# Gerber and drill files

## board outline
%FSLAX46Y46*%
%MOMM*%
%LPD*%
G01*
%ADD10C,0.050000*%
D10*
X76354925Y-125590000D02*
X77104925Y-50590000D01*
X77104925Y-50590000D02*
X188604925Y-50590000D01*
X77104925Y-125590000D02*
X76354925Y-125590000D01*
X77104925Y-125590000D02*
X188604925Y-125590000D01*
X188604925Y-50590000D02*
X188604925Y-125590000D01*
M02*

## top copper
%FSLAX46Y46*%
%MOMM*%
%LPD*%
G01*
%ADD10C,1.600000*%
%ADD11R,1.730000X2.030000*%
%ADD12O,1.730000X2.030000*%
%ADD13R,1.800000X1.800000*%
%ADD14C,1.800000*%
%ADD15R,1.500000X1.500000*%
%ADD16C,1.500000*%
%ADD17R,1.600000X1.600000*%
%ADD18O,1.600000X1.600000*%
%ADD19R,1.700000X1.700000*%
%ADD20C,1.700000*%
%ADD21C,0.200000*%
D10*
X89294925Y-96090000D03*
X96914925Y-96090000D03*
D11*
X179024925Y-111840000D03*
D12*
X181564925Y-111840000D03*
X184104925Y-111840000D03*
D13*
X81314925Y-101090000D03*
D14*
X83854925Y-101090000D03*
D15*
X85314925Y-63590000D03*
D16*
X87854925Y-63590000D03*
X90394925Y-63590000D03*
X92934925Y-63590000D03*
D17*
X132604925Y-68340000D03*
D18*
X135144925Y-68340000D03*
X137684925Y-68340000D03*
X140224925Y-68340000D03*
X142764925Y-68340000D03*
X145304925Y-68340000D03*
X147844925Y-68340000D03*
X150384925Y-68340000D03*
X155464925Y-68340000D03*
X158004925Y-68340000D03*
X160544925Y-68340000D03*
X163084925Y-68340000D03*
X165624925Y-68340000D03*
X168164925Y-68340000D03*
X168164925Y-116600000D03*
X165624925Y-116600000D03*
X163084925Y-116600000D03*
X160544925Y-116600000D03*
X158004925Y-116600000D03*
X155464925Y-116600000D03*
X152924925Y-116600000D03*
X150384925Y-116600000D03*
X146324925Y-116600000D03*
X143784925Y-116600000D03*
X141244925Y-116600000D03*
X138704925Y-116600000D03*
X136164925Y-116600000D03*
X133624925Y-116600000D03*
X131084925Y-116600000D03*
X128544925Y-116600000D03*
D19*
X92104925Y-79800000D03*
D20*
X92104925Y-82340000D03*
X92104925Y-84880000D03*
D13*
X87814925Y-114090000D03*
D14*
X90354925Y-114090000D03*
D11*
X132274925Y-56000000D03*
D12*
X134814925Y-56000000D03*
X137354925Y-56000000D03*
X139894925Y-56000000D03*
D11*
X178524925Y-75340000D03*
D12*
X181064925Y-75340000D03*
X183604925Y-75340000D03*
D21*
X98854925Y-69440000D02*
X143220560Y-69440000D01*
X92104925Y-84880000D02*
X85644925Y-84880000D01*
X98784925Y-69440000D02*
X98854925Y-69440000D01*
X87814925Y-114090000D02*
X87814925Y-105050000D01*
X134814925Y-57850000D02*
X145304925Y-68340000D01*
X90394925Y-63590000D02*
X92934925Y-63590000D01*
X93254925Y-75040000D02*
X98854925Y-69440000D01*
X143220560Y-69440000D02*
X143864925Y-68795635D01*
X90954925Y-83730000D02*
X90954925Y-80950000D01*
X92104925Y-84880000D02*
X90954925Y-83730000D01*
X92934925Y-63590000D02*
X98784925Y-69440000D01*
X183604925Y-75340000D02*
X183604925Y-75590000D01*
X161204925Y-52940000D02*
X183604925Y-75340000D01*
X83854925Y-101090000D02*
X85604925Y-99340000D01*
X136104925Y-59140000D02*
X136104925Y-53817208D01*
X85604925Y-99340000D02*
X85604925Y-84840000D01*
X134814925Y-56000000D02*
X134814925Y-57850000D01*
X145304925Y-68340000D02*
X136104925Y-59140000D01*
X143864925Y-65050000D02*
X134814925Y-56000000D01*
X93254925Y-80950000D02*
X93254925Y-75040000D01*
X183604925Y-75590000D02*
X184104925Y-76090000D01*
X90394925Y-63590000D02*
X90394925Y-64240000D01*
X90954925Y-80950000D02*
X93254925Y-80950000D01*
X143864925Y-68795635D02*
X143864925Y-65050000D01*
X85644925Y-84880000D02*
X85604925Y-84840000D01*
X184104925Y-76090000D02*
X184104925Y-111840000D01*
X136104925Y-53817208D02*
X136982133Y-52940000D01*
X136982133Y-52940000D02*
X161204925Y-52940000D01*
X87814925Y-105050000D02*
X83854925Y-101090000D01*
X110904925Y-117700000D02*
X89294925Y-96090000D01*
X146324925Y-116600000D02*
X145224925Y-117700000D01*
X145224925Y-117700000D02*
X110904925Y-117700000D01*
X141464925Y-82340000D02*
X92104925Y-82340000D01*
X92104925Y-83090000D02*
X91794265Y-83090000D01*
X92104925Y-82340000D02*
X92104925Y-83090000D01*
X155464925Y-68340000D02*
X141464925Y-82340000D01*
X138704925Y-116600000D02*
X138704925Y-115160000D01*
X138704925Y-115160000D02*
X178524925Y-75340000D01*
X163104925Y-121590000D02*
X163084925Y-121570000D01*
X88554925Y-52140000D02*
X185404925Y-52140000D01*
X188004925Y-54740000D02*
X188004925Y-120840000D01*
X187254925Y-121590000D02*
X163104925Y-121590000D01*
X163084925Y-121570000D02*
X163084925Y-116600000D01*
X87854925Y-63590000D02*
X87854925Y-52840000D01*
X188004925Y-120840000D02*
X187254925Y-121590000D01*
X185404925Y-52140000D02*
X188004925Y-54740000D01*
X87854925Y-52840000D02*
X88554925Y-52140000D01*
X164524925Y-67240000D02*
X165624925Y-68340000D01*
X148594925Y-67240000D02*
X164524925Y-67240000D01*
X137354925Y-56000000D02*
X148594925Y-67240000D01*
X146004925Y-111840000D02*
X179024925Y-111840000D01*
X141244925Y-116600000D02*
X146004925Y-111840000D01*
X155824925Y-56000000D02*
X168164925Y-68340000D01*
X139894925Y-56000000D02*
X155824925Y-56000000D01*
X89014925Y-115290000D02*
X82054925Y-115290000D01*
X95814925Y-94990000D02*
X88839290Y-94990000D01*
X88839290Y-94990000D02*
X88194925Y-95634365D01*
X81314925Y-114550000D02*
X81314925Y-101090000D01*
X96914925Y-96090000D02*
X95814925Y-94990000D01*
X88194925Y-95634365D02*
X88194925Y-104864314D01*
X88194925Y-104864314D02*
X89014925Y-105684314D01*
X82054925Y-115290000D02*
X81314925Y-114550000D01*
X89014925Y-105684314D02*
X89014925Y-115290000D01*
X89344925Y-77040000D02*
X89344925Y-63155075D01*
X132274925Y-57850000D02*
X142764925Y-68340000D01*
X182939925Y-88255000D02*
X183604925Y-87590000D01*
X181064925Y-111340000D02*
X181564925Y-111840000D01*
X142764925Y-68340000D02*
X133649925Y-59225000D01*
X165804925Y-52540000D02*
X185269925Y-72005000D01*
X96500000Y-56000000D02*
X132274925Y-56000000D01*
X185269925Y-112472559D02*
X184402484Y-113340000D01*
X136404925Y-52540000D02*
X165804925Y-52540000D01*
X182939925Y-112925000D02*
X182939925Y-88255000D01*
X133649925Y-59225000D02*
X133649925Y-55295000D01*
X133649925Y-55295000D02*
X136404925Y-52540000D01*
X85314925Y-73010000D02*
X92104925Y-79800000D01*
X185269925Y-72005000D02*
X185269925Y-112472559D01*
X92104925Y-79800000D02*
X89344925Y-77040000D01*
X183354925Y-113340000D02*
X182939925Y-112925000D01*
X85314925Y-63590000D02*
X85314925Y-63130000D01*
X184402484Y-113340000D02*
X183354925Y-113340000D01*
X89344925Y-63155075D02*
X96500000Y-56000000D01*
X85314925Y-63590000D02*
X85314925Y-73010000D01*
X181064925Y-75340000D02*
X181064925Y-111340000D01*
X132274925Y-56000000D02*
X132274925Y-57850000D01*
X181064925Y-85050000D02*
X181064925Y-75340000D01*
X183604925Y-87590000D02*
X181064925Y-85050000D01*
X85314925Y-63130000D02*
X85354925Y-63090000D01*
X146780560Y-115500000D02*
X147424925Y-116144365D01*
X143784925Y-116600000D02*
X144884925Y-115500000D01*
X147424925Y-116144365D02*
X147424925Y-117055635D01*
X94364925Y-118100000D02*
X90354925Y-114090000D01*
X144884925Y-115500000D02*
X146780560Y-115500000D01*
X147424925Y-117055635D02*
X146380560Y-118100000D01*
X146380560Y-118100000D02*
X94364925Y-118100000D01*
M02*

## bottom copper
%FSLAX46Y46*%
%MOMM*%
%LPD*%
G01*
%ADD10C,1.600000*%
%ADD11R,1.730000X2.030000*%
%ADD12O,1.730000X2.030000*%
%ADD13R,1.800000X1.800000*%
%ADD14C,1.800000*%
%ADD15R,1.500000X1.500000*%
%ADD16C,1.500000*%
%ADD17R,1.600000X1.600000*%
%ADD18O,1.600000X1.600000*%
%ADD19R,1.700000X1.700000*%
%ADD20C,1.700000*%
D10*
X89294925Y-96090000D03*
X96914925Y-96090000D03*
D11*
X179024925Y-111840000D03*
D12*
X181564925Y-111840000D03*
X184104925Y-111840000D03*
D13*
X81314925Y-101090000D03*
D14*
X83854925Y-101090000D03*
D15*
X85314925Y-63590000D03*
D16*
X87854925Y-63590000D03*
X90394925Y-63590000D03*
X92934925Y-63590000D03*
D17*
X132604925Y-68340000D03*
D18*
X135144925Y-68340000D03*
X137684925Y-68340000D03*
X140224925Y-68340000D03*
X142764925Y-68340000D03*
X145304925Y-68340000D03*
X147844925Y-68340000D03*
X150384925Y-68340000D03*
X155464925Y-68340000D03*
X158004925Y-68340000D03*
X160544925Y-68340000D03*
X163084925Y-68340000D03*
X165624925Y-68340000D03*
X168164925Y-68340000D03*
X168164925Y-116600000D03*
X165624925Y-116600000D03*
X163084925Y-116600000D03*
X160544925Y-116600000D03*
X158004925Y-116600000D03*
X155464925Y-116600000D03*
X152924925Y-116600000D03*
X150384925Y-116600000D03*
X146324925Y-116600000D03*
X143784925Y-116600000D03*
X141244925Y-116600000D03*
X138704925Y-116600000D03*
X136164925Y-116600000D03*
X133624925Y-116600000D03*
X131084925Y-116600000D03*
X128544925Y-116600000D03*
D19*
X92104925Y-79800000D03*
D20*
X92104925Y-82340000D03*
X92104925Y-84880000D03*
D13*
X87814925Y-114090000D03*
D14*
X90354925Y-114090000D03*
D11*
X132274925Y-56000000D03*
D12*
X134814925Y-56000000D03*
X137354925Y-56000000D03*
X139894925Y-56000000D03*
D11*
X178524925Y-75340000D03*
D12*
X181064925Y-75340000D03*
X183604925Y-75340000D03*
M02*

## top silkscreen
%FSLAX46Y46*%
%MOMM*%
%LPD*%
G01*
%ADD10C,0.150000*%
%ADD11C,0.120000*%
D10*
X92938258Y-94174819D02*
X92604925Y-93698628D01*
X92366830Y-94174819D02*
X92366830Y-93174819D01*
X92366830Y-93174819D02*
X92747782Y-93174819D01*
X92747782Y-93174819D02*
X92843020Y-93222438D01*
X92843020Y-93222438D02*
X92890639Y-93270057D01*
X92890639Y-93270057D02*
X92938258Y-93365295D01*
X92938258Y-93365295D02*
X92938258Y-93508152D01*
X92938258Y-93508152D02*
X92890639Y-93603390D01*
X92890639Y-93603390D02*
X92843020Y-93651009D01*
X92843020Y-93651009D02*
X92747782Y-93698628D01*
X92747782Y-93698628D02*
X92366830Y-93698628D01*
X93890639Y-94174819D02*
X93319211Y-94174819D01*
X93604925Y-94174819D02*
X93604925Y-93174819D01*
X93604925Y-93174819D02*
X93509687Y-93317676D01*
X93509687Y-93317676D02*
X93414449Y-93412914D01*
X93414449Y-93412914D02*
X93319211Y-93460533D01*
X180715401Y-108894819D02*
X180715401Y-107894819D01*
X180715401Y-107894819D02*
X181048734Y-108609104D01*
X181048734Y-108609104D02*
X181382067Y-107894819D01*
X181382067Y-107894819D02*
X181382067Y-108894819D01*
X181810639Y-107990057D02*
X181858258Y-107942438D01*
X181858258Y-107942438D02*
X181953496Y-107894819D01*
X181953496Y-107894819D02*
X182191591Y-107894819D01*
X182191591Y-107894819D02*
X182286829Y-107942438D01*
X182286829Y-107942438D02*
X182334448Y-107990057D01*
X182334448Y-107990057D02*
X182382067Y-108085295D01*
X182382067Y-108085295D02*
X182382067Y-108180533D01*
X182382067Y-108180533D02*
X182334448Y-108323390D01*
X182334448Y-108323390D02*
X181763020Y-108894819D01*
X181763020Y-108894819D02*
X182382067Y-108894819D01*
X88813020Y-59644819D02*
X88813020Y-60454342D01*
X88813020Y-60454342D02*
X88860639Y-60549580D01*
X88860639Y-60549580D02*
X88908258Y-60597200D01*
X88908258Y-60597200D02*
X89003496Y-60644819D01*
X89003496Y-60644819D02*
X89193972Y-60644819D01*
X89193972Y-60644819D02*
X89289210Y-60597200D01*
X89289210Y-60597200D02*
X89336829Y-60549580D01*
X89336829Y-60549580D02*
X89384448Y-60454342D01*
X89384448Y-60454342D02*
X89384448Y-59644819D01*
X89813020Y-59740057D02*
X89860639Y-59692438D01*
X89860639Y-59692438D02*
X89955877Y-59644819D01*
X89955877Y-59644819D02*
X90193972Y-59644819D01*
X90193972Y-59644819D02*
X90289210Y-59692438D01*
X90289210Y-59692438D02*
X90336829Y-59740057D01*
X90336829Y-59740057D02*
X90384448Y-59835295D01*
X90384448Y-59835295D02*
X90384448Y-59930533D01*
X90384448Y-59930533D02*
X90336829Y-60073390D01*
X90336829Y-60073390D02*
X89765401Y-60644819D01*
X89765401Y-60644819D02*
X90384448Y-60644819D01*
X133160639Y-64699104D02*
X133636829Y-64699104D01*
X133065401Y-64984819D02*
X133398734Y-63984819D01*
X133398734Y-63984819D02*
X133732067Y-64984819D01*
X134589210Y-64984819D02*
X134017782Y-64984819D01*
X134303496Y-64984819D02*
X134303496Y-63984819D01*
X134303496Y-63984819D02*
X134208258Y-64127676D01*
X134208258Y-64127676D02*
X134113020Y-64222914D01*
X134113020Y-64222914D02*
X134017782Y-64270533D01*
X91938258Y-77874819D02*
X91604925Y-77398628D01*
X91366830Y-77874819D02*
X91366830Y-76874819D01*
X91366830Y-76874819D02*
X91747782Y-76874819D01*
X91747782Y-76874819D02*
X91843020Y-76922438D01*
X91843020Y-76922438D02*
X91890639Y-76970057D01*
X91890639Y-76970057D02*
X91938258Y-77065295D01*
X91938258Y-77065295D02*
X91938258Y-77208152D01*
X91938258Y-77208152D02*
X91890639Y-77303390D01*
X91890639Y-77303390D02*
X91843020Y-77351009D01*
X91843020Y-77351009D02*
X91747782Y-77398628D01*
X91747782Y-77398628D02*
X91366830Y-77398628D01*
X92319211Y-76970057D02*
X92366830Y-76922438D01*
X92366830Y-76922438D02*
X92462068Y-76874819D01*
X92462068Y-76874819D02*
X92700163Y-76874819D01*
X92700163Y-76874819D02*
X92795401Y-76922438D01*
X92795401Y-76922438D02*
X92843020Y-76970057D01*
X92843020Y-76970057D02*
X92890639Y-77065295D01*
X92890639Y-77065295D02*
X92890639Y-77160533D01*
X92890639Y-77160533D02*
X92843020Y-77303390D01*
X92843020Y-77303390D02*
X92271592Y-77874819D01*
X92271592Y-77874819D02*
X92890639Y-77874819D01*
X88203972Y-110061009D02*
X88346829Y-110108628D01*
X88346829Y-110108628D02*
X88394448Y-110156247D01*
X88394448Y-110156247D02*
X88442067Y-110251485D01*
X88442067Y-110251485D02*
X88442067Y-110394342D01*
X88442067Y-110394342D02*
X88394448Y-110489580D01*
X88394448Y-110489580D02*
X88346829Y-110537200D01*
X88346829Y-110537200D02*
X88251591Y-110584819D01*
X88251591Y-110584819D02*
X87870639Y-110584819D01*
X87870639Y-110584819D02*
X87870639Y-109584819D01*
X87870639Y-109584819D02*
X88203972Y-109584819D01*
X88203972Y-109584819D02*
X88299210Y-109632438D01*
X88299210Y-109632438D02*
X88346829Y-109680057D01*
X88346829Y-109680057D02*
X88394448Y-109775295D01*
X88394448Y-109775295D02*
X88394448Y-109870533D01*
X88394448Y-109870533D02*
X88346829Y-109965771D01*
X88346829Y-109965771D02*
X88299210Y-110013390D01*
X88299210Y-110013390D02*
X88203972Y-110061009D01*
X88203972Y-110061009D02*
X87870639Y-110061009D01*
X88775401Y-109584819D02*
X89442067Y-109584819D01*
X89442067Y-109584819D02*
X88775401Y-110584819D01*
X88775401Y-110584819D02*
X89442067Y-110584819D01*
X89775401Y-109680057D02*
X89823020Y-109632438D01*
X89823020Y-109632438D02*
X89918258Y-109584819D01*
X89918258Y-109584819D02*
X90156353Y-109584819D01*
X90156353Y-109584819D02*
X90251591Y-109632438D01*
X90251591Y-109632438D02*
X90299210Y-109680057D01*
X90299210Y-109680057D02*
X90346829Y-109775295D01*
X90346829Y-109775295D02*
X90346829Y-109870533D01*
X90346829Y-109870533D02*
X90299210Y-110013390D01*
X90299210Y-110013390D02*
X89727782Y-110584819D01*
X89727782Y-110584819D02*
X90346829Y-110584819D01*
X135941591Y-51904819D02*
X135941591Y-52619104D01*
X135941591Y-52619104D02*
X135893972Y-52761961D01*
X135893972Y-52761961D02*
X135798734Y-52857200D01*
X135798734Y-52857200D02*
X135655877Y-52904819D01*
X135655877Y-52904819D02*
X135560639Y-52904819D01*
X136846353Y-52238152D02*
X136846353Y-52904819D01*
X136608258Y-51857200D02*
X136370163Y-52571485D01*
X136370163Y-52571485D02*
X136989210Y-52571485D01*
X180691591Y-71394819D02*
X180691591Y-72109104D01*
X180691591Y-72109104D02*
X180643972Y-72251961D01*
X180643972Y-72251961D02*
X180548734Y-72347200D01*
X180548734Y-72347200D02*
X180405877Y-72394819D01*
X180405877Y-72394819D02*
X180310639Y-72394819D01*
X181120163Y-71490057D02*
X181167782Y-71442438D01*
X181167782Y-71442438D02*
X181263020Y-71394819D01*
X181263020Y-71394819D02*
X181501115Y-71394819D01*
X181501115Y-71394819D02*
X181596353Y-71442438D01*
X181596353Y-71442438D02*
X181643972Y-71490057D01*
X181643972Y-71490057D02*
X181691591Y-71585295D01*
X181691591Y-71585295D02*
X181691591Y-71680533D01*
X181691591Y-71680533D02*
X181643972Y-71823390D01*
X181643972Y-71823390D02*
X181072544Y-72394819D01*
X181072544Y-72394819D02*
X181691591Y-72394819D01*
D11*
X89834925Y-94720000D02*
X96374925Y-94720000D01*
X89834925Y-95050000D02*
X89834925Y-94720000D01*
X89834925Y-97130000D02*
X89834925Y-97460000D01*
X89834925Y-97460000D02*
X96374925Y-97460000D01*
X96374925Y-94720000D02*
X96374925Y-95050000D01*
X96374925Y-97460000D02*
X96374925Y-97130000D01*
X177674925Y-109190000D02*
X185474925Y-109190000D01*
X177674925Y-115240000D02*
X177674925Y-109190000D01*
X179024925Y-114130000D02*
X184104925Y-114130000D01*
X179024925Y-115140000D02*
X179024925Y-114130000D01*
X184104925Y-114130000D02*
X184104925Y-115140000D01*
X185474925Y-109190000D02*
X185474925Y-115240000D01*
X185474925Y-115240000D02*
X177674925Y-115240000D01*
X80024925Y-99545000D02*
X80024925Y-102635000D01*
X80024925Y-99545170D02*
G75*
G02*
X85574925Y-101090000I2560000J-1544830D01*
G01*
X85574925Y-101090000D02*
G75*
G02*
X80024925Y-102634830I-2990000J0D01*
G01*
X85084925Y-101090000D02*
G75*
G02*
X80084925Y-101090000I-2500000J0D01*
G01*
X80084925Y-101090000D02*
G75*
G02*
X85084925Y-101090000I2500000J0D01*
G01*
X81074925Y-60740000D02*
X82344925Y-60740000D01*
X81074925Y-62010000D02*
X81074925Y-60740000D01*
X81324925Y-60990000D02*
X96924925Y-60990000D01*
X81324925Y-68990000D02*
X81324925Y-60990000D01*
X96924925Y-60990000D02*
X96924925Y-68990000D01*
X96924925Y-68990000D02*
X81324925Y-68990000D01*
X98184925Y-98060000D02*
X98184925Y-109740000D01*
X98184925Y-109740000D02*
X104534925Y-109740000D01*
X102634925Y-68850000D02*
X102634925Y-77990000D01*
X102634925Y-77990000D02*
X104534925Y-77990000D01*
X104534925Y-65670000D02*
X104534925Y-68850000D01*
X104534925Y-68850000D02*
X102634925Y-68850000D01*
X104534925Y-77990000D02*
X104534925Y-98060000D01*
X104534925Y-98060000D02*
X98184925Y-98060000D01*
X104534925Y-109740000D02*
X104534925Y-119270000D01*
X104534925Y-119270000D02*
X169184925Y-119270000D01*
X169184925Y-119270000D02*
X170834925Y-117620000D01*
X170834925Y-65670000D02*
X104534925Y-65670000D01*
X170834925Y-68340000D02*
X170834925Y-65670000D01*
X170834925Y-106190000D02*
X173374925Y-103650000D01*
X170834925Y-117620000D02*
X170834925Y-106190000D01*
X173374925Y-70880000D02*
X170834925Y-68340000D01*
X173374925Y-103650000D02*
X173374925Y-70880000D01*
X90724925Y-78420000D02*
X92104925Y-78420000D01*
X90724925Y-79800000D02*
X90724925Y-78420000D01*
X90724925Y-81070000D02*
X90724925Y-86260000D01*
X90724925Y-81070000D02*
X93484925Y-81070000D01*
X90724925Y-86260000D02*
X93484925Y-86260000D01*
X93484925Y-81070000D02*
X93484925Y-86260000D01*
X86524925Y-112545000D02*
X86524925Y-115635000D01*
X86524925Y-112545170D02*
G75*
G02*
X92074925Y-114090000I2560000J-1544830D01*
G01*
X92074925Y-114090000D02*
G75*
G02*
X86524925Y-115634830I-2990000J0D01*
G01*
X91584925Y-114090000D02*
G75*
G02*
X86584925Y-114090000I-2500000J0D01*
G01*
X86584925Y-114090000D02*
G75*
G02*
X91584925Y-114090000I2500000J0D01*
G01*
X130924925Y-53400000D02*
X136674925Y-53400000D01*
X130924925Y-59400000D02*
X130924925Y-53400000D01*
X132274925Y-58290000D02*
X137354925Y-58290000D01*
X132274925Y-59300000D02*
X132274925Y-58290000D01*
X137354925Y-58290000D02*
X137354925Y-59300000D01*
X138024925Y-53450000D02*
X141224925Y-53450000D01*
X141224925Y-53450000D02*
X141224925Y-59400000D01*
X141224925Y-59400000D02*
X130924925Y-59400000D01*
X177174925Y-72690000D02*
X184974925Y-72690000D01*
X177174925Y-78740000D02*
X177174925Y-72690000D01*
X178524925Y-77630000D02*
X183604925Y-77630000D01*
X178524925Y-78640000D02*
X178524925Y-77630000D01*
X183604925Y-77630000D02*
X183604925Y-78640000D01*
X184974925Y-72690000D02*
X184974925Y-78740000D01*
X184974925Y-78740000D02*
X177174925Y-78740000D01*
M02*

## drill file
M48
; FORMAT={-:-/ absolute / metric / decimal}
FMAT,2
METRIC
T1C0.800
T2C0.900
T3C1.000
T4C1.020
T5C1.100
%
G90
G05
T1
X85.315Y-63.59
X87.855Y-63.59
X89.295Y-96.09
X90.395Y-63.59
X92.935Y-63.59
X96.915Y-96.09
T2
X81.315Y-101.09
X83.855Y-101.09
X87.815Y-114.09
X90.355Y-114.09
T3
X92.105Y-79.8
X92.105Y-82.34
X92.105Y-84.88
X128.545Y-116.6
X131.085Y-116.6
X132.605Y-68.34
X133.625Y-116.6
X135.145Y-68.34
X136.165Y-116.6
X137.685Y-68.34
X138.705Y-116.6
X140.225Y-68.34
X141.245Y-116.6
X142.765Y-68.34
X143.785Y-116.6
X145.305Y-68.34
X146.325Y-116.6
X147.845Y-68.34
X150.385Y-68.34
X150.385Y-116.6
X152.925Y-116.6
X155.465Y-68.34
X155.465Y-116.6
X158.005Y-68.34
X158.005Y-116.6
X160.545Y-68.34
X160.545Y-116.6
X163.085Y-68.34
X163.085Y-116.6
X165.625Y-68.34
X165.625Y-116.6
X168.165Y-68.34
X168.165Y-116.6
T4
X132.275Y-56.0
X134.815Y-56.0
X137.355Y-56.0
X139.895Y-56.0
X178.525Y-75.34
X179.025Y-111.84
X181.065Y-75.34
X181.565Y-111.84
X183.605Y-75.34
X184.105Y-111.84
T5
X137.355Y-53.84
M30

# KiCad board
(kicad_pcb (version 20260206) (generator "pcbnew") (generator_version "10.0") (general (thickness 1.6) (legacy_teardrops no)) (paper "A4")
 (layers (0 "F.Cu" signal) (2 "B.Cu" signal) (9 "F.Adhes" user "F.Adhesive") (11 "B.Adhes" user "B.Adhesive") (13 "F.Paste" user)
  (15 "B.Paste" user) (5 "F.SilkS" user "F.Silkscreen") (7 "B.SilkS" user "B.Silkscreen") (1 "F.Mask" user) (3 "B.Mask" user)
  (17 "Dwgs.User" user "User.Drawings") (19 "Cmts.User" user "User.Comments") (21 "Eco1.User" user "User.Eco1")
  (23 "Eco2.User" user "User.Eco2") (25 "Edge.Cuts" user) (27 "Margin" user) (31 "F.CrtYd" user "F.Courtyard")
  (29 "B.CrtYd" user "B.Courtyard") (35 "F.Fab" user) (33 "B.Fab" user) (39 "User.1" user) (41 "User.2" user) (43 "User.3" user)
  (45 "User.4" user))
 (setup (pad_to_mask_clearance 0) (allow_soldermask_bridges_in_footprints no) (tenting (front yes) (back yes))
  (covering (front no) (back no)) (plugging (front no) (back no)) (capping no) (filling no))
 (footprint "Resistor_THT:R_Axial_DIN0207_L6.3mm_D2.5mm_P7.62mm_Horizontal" (layer "F.Cu") (at 89.294925 96.09)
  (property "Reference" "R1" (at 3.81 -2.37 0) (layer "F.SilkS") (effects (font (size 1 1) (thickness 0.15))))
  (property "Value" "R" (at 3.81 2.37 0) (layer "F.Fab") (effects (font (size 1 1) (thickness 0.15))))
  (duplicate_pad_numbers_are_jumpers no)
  (fp_line (start 0.54 -1.37) (end 7.08 -1.37) (stroke (width 0.12) (type solid)) (layer "F.SilkS"))
  (fp_line (start 0.54 -1.04) (end 0.54 -1.37) (stroke (width 0.12) (type solid)) (layer "F.SilkS"))
  (fp_line (start 0.54 1.04) (end 0.54 1.37) (stroke (width 0.12) (type solid)) (layer "F.SilkS"))
  (fp_line (start 0.54 1.37) (end 7.08 1.37) (stroke (width 0.12) (type solid)) (layer "F.SilkS"))
  (fp_line (start 7.08 -1.37) (end 7.08 -1.04) (stroke (width 0.12) (type solid)) (layer "F.SilkS"))
  (fp_line (start 7.08 1.37) (end 7.08 1.04) (stroke (width 0.12) (type solid)) (layer "F.SilkS"))
  (pad "1" thru_hole circle (at 0 0) (size 1.6 1.6) (drill 0.8) (layers "*.Cu" "*.Mask") (remove_unused_layers no) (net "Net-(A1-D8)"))
  (pad "2" thru_hole circle (at 7.62 0) (size 1.6 1.6) (drill 0.8) (layers "*.Cu" "*.Mask") (remove_unused_layers no) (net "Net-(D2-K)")))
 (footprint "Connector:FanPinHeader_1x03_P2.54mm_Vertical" (layer "F.Cu") (at 179.024925 111.84)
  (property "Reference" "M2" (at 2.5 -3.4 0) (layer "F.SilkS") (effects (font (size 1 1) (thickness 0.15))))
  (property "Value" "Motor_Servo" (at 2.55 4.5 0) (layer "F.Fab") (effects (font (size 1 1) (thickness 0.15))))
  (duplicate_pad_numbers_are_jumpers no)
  (fp_line (start -1.35 -2.65) (end 6.45 -2.65) (stroke (width 0.12) (type solid)) (layer "F.SilkS"))
  (fp_line (start -1.35 3.4) (end -1.35 -2.65) (stroke (width 0.12) (type solid)) (layer "F.SilkS"))
  (fp_line (start 0 2.29) (end 5.08 2.29) (stroke (width 0.12) (type solid)) (layer "F.SilkS"))
  (fp_line (start 0 3.3) (end 0 2.29) (stroke (width 0.12) (type solid)) (layer "F.SilkS"))
  (fp_line (start 5.08 2.29) (end 5.08 3.3) (stroke (width 0.12) (type solid)) (layer "F.SilkS"))
  (fp_line (start 6.45 -2.65) (end 6.45 3.4) (stroke (width 0.12) (type solid)) (layer "F.SilkS"))
  (fp_line (start 6.45 3.4) (end -1.35 3.4) (stroke (width 0.12) (type solid)) (layer "F.SilkS"))
  (pad "1" thru_hole rect (at 0 0 90) (size 2.03 1.73) (drill 1.02) (layers "*.Cu" "*.Mask") (remove_unused_layers no) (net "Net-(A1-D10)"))
  (pad "2" thru_hole oval (at 2.54 0 90) (size 2.03 1.73) (drill 1.02) (layers "*.Cu" "*.Mask") (remove_unused_layers no) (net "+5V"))
  (pad "3" thru_hole oval (at 5.08 0 90) (size 2.03 1.73) (drill 1.02) (layers "*.Cu" "*.Mask") (remove_unused_layers no) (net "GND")))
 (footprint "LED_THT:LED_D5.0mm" (layer "F.Cu") (at 81.314925 101.09)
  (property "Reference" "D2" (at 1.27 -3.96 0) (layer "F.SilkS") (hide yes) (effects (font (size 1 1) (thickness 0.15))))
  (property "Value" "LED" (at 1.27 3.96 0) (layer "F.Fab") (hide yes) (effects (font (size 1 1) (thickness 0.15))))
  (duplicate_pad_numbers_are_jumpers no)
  (fp_line (start -1.29 -1.545) (end -1.29 1.545) (stroke (width 0.12) (type solid)) (layer "F.SilkS"))
  (fp_arc (start -1.29 -1.54483) (mid 2.071779 -2.880495) (end 4.26 0) (stroke (width 0.12) (type solid)) (layer "F.SilkS"))
  (fp_arc (start 4.26 0) (mid 2.071779 2.880495) (end -1.29 1.54483) (stroke (width 0.12) (type solid)) (layer "F.SilkS"))
  (fp_circle (center 1.27 0) (end 3.77 0) (stroke (width 0.12) (type solid)) (fill no) (layer "F.SilkS"))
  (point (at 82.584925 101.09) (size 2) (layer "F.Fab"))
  (pad "1" thru_hole rect (at 0 0) (size 1.8 1.8) (drill 0.9) (layers "*.Cu" "*.Mask") (remove_unused_layers no) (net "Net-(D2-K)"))
  (pad "2" thru_hole circle (at 2.54 0) (size 1.8 1.8) (drill 0.9) (layers "*.Cu" "*.Mask") (remove_unused_layers no) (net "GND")))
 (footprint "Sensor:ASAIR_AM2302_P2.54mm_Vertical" (layer "F.Cu") (at 85.314925 63.59)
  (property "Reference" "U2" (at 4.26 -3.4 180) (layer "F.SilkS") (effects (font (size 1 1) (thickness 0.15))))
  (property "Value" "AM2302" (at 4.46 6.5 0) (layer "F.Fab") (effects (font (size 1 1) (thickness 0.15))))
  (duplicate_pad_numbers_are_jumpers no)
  (fp_line (start -4.24 -2.85) (end -2.97 -2.85) (stroke (width 0.12) (type solid)) (layer "F.SilkS"))
  (fp_line (start -4.24 -1.58) (end -4.24 -2.85) (stroke (width 0.12) (type solid)) (layer "F.SilkS"))
  (fp_line (start -3.99 -2.6) (end 11.61 -2.6) (stroke (width 0.12) (type solid)) (layer "F.SilkS"))
  (fp_line (start -3.99 5.4) (end -3.99 -2.6) (stroke (width 0.12) (type solid)) (layer "F.SilkS"))
  (fp_line (start 11.61 -2.6) (end 11.61 5.4) (stroke (width 0.12) (type solid)) (layer "F.SilkS"))
  (fp_line (start 11.61 5.4) (end -3.99 5.4) (stroke (width 0.12) (type solid)) (layer "F.SilkS"))
  (pad "1" thru_hole rect (at 0 0 90) (size 1.5 1.5) (drill 0.8) (layers "*.Cu" "*.Mask") (remove_unused_layers no) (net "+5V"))
  (pad "2" thru_hole circle (at 2.54 0 90) (size 1.5 1.5) (drill 0.8) (layers "*.Cu" "*.Mask") (remove_unused_layers no) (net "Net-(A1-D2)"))
  (pad "3" thru_hole circle (at 5.08 0 90) (size 1.5 1.5) (drill 0.8) (layers "*.Cu" "*.Mask") (remove_unused_layers no) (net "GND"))
  (pad "4" thru_hole circle (at 7.62 0 90) (size 1.5 1.5) (drill 0.8) (layers "*.Cu" "*.Mask") (remove_unused_layers no) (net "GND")))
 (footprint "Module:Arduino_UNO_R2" (layer "F.Cu") (at 132.604925 68.34)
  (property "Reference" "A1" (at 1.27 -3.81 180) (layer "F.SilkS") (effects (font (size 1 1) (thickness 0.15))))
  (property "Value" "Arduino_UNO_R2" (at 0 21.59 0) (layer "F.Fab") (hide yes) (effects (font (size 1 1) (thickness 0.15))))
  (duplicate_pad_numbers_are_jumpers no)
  (fp_line (start -34.42 29.72) (end -34.42 41.4) (stroke (width 0.12) (type solid)) (layer "F.SilkS"))
  (fp_line (start -34.42 41.4) (end -28.07 41.4) (stroke (width 0.12) (type solid)) (layer "F.SilkS"))
  (fp_line (start -29.97 0.51) (end -29.97 9.65) (stroke (width 0.12) (type solid)) (layer "F.SilkS"))
  (fp_line (start -29.97 9.65) (end -28.07 9.65) (stroke (width 0.12) (type solid)) (layer "F.SilkS"))
  (fp_line (start -28.07 -2.67) (end -28.07 0.51) (stroke (width 0.12) (type solid)) (layer "F.SilkS"))
  (fp_line (start -28.07 0.51) (end -29.97 0.51) (stroke (width 0.12) (type solid)) (layer "F.SilkS"))
  (fp_line (start -28.07 9.65) (end -28.07 29.72) (stroke (width 0.12) (type solid)) (layer "F.SilkS"))
  (fp_line (start -28.07 29.72) (end -34.42 29.72) (stroke (width 0.12) (type solid)) (layer "F.SilkS"))
  (fp_line (start -28.07 41.4) (end -28.07 50.93) (stroke (width 0.12) (type solid)) (layer "F.SilkS"))
  (fp_line (start -28.07 50.93) (end 36.58 50.93) (stroke (width 0.12) (type solid)) (layer "F.SilkS"))
  (fp_line (start 36.58 50.93) (end 38.23 49.28) (stroke (width 0.12) (type solid)) (layer "F.SilkS"))
  (fp_line (start 38.23 -2.67) (end -28.07 -2.67) (stroke (width 0.12) (type solid)) (layer "F.SilkS"))
  (fp_line (start 38.23 0) (end 38.23 -2.67) (stroke (width 0.12) (type solid)) (layer "F.SilkS"))
  (fp_line (start 38.23 37.85) (end 40.77 35.31) (stroke (width 0.12) (type solid)) (layer "F.SilkS"))
  (fp_line (start 38.23 49.28) (end 38.23 37.85) (stroke (width 0.12) (type solid)) (layer "F.SilkS"))
  (fp_line (start 40.77 2.54) (end 38.23 0) (stroke (width 0.12) (type solid)) (layer "F.SilkS"))
  (fp_line (start 40.77 35.31) (end 40.77 2.54) (stroke (width 0.12) (type solid)) (layer "F.SilkS"))
  (pad "1" thru_hole rect (at 0 0 90) (size 1.6 1.6) (drill 1) (layers "*.Cu" "*.Mask") (remove_unused_layers no)
   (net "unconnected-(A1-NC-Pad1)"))
  (pad "2" thru_hole oval (at 2.54 0 90) (size 1.6 1.6) (drill 1) (layers "*.Cu" "*.Mask") (remove_unused_layers no)
   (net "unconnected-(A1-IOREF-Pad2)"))
  (pad "3" thru_hole oval (at 5.08 0 90) (size 1.6 1.6) (drill 1) (layers "*.Cu" "*.Mask") (remove_unused_layers no)
   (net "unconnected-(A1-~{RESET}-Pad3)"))
  (pad "4" thru_hole oval (at 7.62 0 90) (size 1.6 1.6) (drill 1) (layers "*.Cu" "*.Mask") (remove_unused_layers no)
   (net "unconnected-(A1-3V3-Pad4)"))
  (pad "5" thru_hole oval (at 10.16 0 90) (size 1.6 1.6) (drill 1) (layers "*.Cu" "*.Mask") (remove_unused_layers no) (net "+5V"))
  (pad "6" thru_hole oval (at 12.7 0 90) (size 1.6 1.6) (drill 1) (layers "*.Cu" "*.Mask") (remove_unused_layers no) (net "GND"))
  (pad "7" thru_hole oval (at 15.24 0 90) (size 1.6 1.6) (drill 1) (layers "*.Cu" "*.Mask") (remove_unused_layers no)
   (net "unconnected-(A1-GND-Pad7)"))
  (pad "8" thru_hole oval (at 17.78 0 90) (size 1.6 1.6) (drill 1) (layers "*.Cu" "*.Mask") (remove_unused_layers no)
   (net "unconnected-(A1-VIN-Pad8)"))
  (pad "9" thru_hole oval (at 22.86 0 90) (size 1.6 1.6) (drill 1) (layers "*.Cu" "*.Mask") (remove_unused_layers no) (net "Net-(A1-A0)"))
  (pad "10" thru_hole oval (at 25.4 0 90) (size 1.6 1.6) (drill 1) (layers "*.Cu" "*.Mask") (remove_unused_layers no)
   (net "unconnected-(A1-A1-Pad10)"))
  (pad "11" thru_hole oval (at 27.94 0 90) (size 1.6 1.6) (drill 1) (layers "*.Cu" "*.Mask") (remove_unused_layers no)
   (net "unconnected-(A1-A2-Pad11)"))
  (pad "12" thru_hole oval (at 30.48 0 90) (size 1.6 1.6) (drill 1) (layers "*.Cu" "*.Mask") (remove_unused_layers no)
   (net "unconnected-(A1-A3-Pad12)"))
  (pad "13" thru_hole oval (at 33.02 0 90) (size 1.6 1.6) (drill 1) (layers "*.Cu" "*.Mask") (remove_unused_layers no)
   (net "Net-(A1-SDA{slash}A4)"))
  (pad "14" thru_hole oval (at 35.56 0 90) (size 1.6 1.6) (drill 1) (layers "*.Cu" "*.Mask") (remove_unused_layers no)
   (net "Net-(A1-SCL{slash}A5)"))
  (pad "15" thru_hole oval (at 35.56 48.26 90) (size 1.6 1.6) (drill 1) (layers "*.Cu" "*.Mask") (remove_unused_layers no)
   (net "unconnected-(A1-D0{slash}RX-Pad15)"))
  (pad "16" thru_hole oval (at 33.02 48.26 90) (size 1.6 1.6) (drill 1) (layers "*.Cu" "*.Mask") (remove_unused_layers no)
   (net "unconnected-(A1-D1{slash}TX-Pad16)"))
  (pad "17" thru_hole oval (at 30.48 48.26 90) (size 1.6 1.6) (drill 1) (layers "*.Cu" "*.Mask") (remove_unused_layers no)
   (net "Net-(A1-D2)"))
  (pad "18" thru_hole oval (at 27.94 48.26 90) (size 1.6 1.6) (drill 1) (layers "*.Cu" "*.Mask") (remove_unused_layers no)
   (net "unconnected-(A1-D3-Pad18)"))
  (pad "19" thru_hole oval (at 25.4 48.26 90) (size 1.6 1.6) (drill 1) (layers "*.Cu" "*.Mask") (remove_unused_layers no)
   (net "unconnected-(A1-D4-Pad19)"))
  (pad "20" thru_hole oval (at 22.86 48.26 90) (size 1.6 1.6) (drill 1) (layers "*.Cu" "*.Mask") (remove_unused_layers no)
   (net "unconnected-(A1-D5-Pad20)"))
  (pad "21" thru_hole oval (at 20.32 48.26 90) (size 1.6 1.6) (drill 1) (layers "*.Cu" "*.Mask") (remove_unused_layers no)
   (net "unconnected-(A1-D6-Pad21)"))
  (pad "22" thru_hole oval (at 17.78 48.26 90) (size 1.6 1.6) (drill 1) (layers "*.Cu" "*.Mask") (remove_unused_layers no)
   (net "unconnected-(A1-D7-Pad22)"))
  (pad "23" thru_hole oval (at 13.72 48.26 90) (size 1.6 1.6) (drill 1) (layers "*.Cu" "*.Mask") (remove_unused_layers no)
   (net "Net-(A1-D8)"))
  (pad "24" thru_hole oval (at 11.18 48.26 90) (size 1.6 1.6) (drill 1) (layers "*.Cu" "*.Mask") (remove_unused_layers no)
   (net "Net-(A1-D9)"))
  (pad "25" thru_hole oval (at 8.64 48.26 90) (size 1.6 1.6) (drill 1) (layers "*.Cu" "*.Mask") (remove_unused_layers no)
   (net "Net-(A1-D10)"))
  (pad "26" thru_hole oval (at 6.1 48.26 90) (size 1.6 1.6) (drill 1) (layers "*.Cu" "*.Mask") (remove_unused_layers no)
   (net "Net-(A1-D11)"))
  (pad "27" thru_hole oval (at 3.56 48.26 90) (size 1.6 1.6) (drill 1) (layers "*.Cu" "*.Mask") (remove_unused_layers no)
   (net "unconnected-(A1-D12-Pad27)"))
  (pad "28" thru_hole oval (at 1.02 48.26 90) (size 1.6 1.6) (drill 1) (layers "*.Cu" "*.Mask") (remove_unused_layers no)
   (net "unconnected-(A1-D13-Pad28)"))
  (pad "29" thru_hole oval (at -1.52 48.26 90) (size 1.6 1.6) (drill 1) (layers "*.Cu" "*.Mask") (remove_unused_layers no)
   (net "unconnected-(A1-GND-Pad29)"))
  (pad "30" thru_hole oval (at -4.06 48.26 90) (size 1.6 1.6) (drill 1) (layers "*.Cu" "*.Mask") (remove_unused_layers no)
   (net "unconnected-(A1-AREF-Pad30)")))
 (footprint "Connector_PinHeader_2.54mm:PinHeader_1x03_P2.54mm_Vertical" (layer "F.Cu") (at 92.104925 79.8)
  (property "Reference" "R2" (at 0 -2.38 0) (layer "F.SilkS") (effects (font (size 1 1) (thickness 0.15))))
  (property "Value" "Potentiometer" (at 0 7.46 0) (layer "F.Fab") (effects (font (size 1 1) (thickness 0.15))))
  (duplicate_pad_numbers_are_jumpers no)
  (fp_line (start -1.38 -1.38) (end 0 -1.38) (stroke (width 0.12) (type solid)) (layer "F.SilkS"))
  (fp_line (start -1.38 0) (end -1.38 -1.38) (stroke (width 0.12) (type solid)) (layer "F.SilkS"))
  (fp_line (start -1.38 1.27) (end -1.38 6.46) (stroke (width 0.12) (type solid)) (layer "F.SilkS"))
  (fp_line (start -1.38 1.27) (end 1.38 1.27) (stroke (width 0.12) (type solid)) (layer "F.SilkS"))
  (fp_line (start -1.38 6.46) (end 1.38 6.46) (stroke (width 0.12) (type solid)) (layer "F.SilkS"))
  (fp_line (start 1.38 1.27) (end 1.38 6.46) (stroke (width 0.12) (type solid)) (layer "F.SilkS"))
  (pad "1" thru_hole rect (at 0 0) (size 1.7 1.7) (drill 1) (layers "*.Cu" "*.Mask") (remove_unused_layers no) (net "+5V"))
  (pad "2" thru_hole circle (at 0 2.54) (size 1.7 1.7) (drill 1) (layers "*.Cu" "*.Mask") (remove_unused_layers no) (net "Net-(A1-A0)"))
  (pad "3" thru_hole circle (at 0 5.08) (size 1.7 1.7) (drill 1) (layers "*.Cu" "*.Mask") (remove_unused_layers no) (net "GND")))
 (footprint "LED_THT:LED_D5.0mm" (layer "F.Cu") (at 87.814925 114.09)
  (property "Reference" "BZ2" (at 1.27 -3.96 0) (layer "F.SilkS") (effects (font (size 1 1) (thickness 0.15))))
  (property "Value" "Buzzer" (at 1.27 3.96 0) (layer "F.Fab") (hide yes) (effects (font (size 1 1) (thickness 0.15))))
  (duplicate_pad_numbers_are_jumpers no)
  (fp_line (start -1.29 -1.545) (end -1.29 1.545) (stroke (width 0.12) (type solid)) (layer "F.SilkS"))
  (fp_arc (start -1.29 -1.54483) (mid 2.071779 -2.880495) (end 4.26 0) (stroke (width 0.12) (type solid)) (layer "F.SilkS"))
  (fp_arc (start 4.26 0) (mid 2.071779 2.880495) (end -1.29 1.54483) (stroke (width 0.12) (type solid)) (layer "F.SilkS"))
  (fp_circle (center 1.27 0) (end 3.77 0) (stroke (width 0.12) (type solid)) (fill no) (layer "F.SilkS"))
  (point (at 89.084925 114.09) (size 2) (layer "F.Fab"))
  (pad "1" thru_hole rect (at 0 0) (size 1.8 1.8) (drill 0.9) (layers "*.Cu" "*.Mask") (remove_unused_layers no) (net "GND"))
  (pad "2" thru_hole circle (at 2.54 0) (size 1.8 1.8) (drill 0.9) (layers "*.Cu" "*.Mask") (remove_unused_layers no) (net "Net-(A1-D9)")))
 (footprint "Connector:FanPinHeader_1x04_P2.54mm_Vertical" (layer "F.Cu") (at 132.274925 56)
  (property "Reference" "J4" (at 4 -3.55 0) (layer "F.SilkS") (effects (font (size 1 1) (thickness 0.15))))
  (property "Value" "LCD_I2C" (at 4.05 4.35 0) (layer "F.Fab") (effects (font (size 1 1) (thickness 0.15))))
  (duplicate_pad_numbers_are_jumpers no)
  (fp_line (start -1.35 -2.6) (end 4.4 -2.6) (stroke (width 0.12) (type solid)) (layer "F.SilkS"))
  (fp_line (start -1.35 3.4) (end -1.35 -2.6) (stroke (width 0.12) (type solid)) (layer "F.SilkS"))
  (fp_line (start 0 2.29) (end 5.08 2.29) (stroke (width 0.12) (type solid)) (layer "F.SilkS"))
  (fp_line (start 0 3.3) (end 0 2.29) (stroke (width 0.12) (type solid)) (layer "F.SilkS"))
  (fp_line (start 5.08 2.29) (end 5.08 3.3) (stroke (width 0.12) (type solid)) (layer "F.SilkS"))
  (fp_line (start 5.75 -2.55) (end 8.95 -2.55) (stroke (width 0.12) (type solid)) (layer "F.SilkS"))
  (fp_line (start 8.95 -2.55) (end 8.95 3.4) (stroke (width 0.12) (type solid)) (layer "F.SilkS"))
  (fp_line (start 8.95 3.4) (end -1.35 3.4) (stroke (width 0.12) (type solid)) (layer "F.SilkS"))
  (pad "" np_thru_hole circle (at 5.08 -2.16 90) (size 1.1 1.1) (drill 1.1) (layers "*.Cu" "*.Mask"))
  (pad "1" thru_hole rect (at 0 0 90) (size 2.03 1.73) (drill 1.02) (layers "*.Cu" "*.Mask") (remove_unused_layers no) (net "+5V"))
  (pad "2" thru_hole oval (at 2.54 0 90) (size 2.03 1.73) (drill 1.02) (layers "*.Cu" "*.Mask") (remove_unused_layers no) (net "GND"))
  (pad "3" thru_hole oval (at 5.08 0 90) (size 2.03 1.73) (drill 1.02) (layers "*.Cu" "*.Mask") (remove_unused_layers no)
   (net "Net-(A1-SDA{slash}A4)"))
  (pad "4" thru_hole oval (at 7.62 0 90) (size 2.03 1.73) (drill 1.02) (layers "*.Cu" "*.Mask") (remove_unused_layers no)
   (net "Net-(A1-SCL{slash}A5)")))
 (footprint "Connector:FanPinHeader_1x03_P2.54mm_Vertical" (layer "F.Cu") (at 178.524925 75.34)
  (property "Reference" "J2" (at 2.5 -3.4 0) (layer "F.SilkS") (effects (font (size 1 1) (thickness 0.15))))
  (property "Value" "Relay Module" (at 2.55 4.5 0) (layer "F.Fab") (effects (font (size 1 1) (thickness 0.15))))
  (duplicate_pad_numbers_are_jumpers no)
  (fp_line (start -1.35 -2.65) (end 6.45 -2.65) (stroke (width 0.12) (type solid)) (layer "F.SilkS"))
  (fp_line (start -1.35 3.4) (end -1.35 -2.65) (stroke (width 0.12) (type solid)) (layer "F.SilkS"))
  (fp_line (start 0 2.29) (end 5.08 2.29) (stroke (width 0.12) (type solid)) (layer "F.SilkS"))
  (fp_line (start 0 3.3) (end 0 2.29) (stroke (width 0.12) (type solid)) (layer "F.SilkS"))
  (fp_line (start 5.08 2.29) (end 5.08 3.3) (stroke (width 0.12) (type solid)) (layer "F.SilkS"))
  (fp_line (start 6.45 -2.65) (end 6.45 3.4) (stroke (width 0.12) (type solid)) (layer "F.SilkS"))
  (fp_line (start 6.45 3.4) (end -1.35 3.4) (stroke (width 0.12) (type solid)) (layer "F.SilkS"))
  (pad "1" thru_hole rect (at 0 0 90) (size 2.03 1.73) (drill 1.02) (layers "*.Cu" "*.Mask") (remove_unused_layers no) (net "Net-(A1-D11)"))
  (pad "2" thru_hole oval (at 2.54 0 90) (size 2.03 1.73) (drill 1.02) (layers "*.Cu" "*.Mask") (remove_unused_layers no) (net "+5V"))
  (pad "3" thru_hole oval (at 5.08 0 90) (size 2.03 1.73) (drill 1.02) (layers "*.Cu" "*.Mask") (remove_unused_layers no) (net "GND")))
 (gr_line (start 76.354925 125.59) (end 77.104925 50.59) (stroke (width 0.05) (type default)) (layer "Edge.Cuts"))
 (gr_line (start 77.104925 50.59) (end 188.604925 50.59) (stroke (width 0.05) (type default)) (layer "Edge.Cuts"))
 (gr_line (start 77.104925 125.59) (end 76.354925 125.59) (stroke (width 0.05) (type default)) (layer "Edge.Cuts"))
 (gr_line (start 77.104925 125.59) (end 188.604925 125.59) (stroke (width 0.05) (type default)) (layer "Edge.Cuts"))
 (gr_line (start 188.604925 50.59) (end 188.604925 125.59) (stroke (width 0.05) (type default)) (layer "Edge.Cuts"))
 (segment (start 98.854925 69.44) (end 143.22056 69.44) (width 0.2) (layer "F.Cu") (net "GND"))
 (segment (start 92.104925 84.88) (end 85.644925 84.88) (width 0.2) (layer "F.Cu") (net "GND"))
 (segment (start 98.784925 69.44) (end 98.854925 69.44) (width 0.2) (layer "F.Cu") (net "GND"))
 (segment (start 87.814925 114.09) (end 87.814925 105.05) (width 0.2) (layer "F.Cu") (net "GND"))
 (segment (start 134.814925 57.85) (end 145.304925 68.34) (width 0.2) (layer "F.Cu") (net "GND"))
 (segment (start 90.394925 63.59) (end 92.934925 63.59) (width 0.2) (layer "F.Cu") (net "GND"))
 (segment (start 93.254925 75.04) (end 98.854925 69.44) (width 0.2) (layer "F.Cu") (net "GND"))
 (segment (start 143.22056 69.44) (end 143.864925 68.795635) (width 0.2) (layer "F.Cu") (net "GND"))
 (segment (start 90.954925 83.73) (end 90.954925 80.95) (width 0.2) (layer "F.Cu") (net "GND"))
 (segment (start 92.104925 84.88) (end 90.954925 83.73) (width 0.2) (layer "F.Cu") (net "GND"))
 (segment (start 92.934925 63.59) (end 98.784925 69.44) (width 0.2) (layer "F.Cu") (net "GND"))
 (segment (start 183.604925 75.34) (end 183.604925 75.59) (width 0.2) (layer "F.Cu") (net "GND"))
 (segment (start 161.204925 52.94) (end 183.604925 75.34) (width 0.2) (layer "F.Cu") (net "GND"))
 (segment (start 83.854925 101.09) (end 85.604925 99.34) (width 0.2) (layer "F.Cu") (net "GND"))
 (segment (start 136.104925 59.14) (end 136.104925 53.817208) (width 0.2) (layer "F.Cu") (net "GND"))
 (segment (start 85.604925 99.34) (end 85.604925 84.84) (width 0.2) (layer "F.Cu") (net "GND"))
 (segment (start 134.814925 56) (end 134.814925 57.85) (width 0.2) (layer "F.Cu") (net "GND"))
 (segment (start 145.304925 68.34) (end 136.104925 59.14) (width 0.2) (layer "F.Cu") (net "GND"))
 (segment (start 143.864925 65.05) (end 134.814925 56) (width 0.2) (layer "F.Cu") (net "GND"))
 (segment (start 93.254925 80.95) (end 93.254925 75.04) (width 0.2) (layer "F.Cu") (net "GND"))
 (segment (start 183.604925 75.59) (end 184.104925 76.09) (width 0.2) (layer "F.Cu") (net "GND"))
 (segment (start 90.394925 63.59) (end 90.394925 64.24) (width 0.2) (layer "F.Cu") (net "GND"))
 (segment (start 90.954925 80.95) (end 93.254925 80.95) (width 0.2) (layer "F.Cu") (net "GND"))
 (segment (start 143.864925 68.795635) (end 143.864925 65.05) (width 0.2) (layer "F.Cu") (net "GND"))
 (segment (start 85.644925 84.88) (end 85.604925 84.84) (width 0.2) (layer "F.Cu") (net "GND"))
 (segment (start 184.104925 76.09) (end 184.104925 111.84) (width 0.2) (layer "F.Cu") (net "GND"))
 (segment (start 136.104925 53.817208) (end 136.982133 52.94) (width 0.2) (layer "F.Cu") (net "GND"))
 (segment (start 136.982133 52.94) (end 161.204925 52.94) (width 0.2) (layer "F.Cu") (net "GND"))
 (segment (start 87.814925 105.05) (end 83.854925 101.09) (width 0.2) (layer "F.Cu") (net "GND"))
 (segment (start 110.904925 117.7) (end 89.294925 96.09) (width 0.2) (layer "F.Cu") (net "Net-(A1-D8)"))
 (segment (start 146.324925 116.6) (end 145.224925 117.7) (width 0.2) (layer "F.Cu") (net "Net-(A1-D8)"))
 (segment (start 145.224925 117.7) (end 110.904925 117.7) (width 0.2) (layer "F.Cu") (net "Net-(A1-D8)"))
 (segment (start 141.464925 82.34) (end 92.104925 82.34) (width 0.2) (layer "F.Cu") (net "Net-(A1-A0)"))
 (segment (start 92.104925 83.09) (end 91.794265 83.09) (width 0.2) (layer "F.Cu") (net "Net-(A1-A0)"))
 (segment (start 92.104925 82.34) (end 92.104925 83.09) (width 0.2) (layer "F.Cu") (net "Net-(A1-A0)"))
 (segment (start 155.464925 68.34) (end 141.464925 82.34) (width 0.2) (layer "F.Cu") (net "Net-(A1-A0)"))
 (segment (start 138.704925 116.6) (end 138.704925 115.16) (width 0.2) (layer "F.Cu") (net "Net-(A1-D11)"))
 (segment (start 138.704925 115.16) (end 178.524925 75.34) (width 0.2) (layer "F.Cu") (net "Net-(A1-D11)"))
 (segment (start 163.104925 121.59) (end 163.084925 121.57) (width 0.2) (layer "F.Cu") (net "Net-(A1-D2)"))
 (segment (start 88.554925 52.14) (end 185.404925 52.14) (width 0.2) (layer "F.Cu") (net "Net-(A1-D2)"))
 (segment (start 188.004925 54.74) (end 188.004925 120.84) (width 0.2) (layer "F.Cu") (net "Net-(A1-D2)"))
 (segment (start 187.254925 121.59) (end 163.104925 121.59) (width 0.2) (layer "F.Cu") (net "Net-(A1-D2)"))
 (segment (start 163.084925 121.57) (end 163.084925 116.6) (width 0.2) (layer "F.Cu") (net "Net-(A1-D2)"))
 (segment (start 87.854925 63.59) (end 87.854925 52.84) (width 0.2) (layer "F.Cu") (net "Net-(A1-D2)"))
 (segment (start 188.004925 120.84) (end 187.254925 121.59) (width 0.2) (layer "F.Cu") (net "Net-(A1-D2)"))
 (segment (start 185.404925 52.14) (end 188.004925 54.74) (width 0.2) (layer "F.Cu") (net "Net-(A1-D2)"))
 (segment (start 87.854925 52.84) (end 88.554925 52.14) (width 0.2) (layer "F.Cu") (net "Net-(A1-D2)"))
 (segment (start 164.524925 67.24) (end 165.624925 68.34) (width 0.2) (layer "F.Cu") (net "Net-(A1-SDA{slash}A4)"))
 (segment (start 148.594925 67.24) (end 164.524925 67.24) (width 0.2) (layer "F.Cu") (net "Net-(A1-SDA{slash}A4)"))
 (segment (start 137.354925 56) (end 148.594925 67.24) (width 0.2) (layer "F.Cu") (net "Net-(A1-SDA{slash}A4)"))
 (segment (start 146.004925 111.84) (end 179.024925 111.84) (width 0.2) (layer "F.Cu") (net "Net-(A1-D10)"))
 (segment (start 141.244925 116.6) (end 146.004925 111.84) (width 0.2) (layer "F.Cu") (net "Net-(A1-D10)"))
 (segment (start 155.824925 56) (end 168.164925 68.34) (width 0.2) (layer "F.Cu") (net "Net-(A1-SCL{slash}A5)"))
 (segment (start 139.894925 56) (end 155.824925 56) (width 0.2) (layer "F.Cu") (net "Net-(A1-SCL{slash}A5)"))
 (segment (start 89.014925 115.29) (end 82.054925 115.29) (width 0.2) (layer "F.Cu") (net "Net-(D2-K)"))
 (segment (start 95.814925 94.99) (end 88.83929 94.99) (width 0.2) (layer "F.Cu") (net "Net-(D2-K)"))
 (segment (start 88.83929 94.99) (end 88.194925 95.634365) (width 0.2) (layer "F.Cu") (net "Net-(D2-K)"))
 (segment (start 81.314925 114.55) (end 81.314925 101.09) (width 0.2) (layer "F.Cu") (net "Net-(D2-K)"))
 (segment (start 96.914925 96.09) (end 95.814925 94.99) (width 0.2) (layer "F.Cu") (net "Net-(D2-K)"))
 (segment (start 88.194925 95.634365) (end 88.194925 104.864314) (width 0.2) (layer "F.Cu") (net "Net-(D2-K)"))
 (segment (start 88.194925 104.864314) (end 89.014925 105.684314) (width 0.2) (layer "F.Cu") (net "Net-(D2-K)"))
 (segment (start 82.054925 115.29) (end 81.314925 114.55) (width 0.2) (layer "F.Cu") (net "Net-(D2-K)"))
 (segment (start 89.014925 105.684314) (end 89.014925 115.29) (width 0.2) (layer "F.Cu") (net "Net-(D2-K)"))
 (segment (start 89.344925 77.04) (end 89.344925 63.155075) (width 0.2) (layer "F.Cu") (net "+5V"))
 (segment (start 132.274925 57.85) (end 142.764925 68.34) (width 0.2) (layer "F.Cu") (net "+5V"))
 (segment (start 182.939925 88.255) (end 183.604925 87.59) (width 0.2) (layer "F.Cu") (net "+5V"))
 (segment (start 181.064925 111.34) (end 181.564925 111.84) (width 0.2) (layer "F.Cu") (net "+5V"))
 (segment (start 142.764925 68.34) (end 133.649925 59.225) (width 0.2) (layer "F.Cu") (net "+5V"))
 (segment (start 165.804925 52.54) (end 185.269925 72.005) (width 0.2) (layer "F.Cu") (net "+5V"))
 (segment (start 96.5 56) (end 132.274925 56) (width 0.2) (layer "F.Cu") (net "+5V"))
 (segment (start 185.269925 112.472559) (end 184.402484 113.34) (width 0.2) (layer "F.Cu") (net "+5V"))
 (segment (start 136.404925 52.54) (end 165.804925 52.54) (width 0.2) (layer "F.Cu") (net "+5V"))
 (segment (start 182.939925 112.925) (end 182.939925 88.255) (width 0.2) (layer "F.Cu") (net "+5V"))
 (segment (start 133.649925 59.225) (end 133.649925 55.295) (width 0.2) (layer "F.Cu") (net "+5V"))
 (segment (start 133.649925 55.295) (end 136.404925 52.54) (width 0.2) (layer "F.Cu") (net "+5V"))
 (segment (start 85.314925 73.01) (end 92.104925 79.8) (width 0.2) (layer "F.Cu") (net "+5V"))
 (segment (start 185.269925 72.005) (end 185.269925 112.472559) (width 0.2) (layer "F.Cu") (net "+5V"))
 (segment (start 92.104925 79.8) (end 89.344925 77.04) (width 0.2) (layer "F.Cu") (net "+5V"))
 (segment (start 183.354925 113.34) (end 182.939925 112.925) (width 0.2) (layer "F.Cu") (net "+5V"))
 (segment (start 85.314925 63.59) (end 85.314925 63.13) (width 0.2) (layer "F.Cu") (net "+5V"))
 (segment (start 184.402484 113.34) (end 183.354925 113.34) (width 0.2) (layer "F.Cu") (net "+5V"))
 (segment (start 89.344925 63.155075) (end 96.5 56) (width 0.2) (layer "F.Cu") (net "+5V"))
 (segment (start 85.314925 63.59) (end 85.314925 73.01) (width 0.2) (layer "F.Cu") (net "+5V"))
 (segment (start 181.064925 75.34) (end 181.064925 111.34) (width 0.2) (layer "F.Cu") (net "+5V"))
 (segment (start 132.274925 56) (end 132.274925 57.85) (width 0.2) (layer "F.Cu") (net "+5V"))
 (segment (start 181.064925 85.05) (end 181.064925 75.34) (width 0.2) (layer "F.Cu") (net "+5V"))
 (segment (start 183.604925 87.59) (end 181.064925 85.05) (width 0.2) (layer "F.Cu") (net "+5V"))
 (segment (start 85.314925 63.13) (end 85.354925 63.09) (width 0.2) (layer "F.Cu") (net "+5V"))
 (segment (start 146.78056 115.5) (end 147.424925 116.144365) (width 0.2) (layer "F.Cu") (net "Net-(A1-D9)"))
 (segment (start 143.784925 116.6) (end 144.884925 115.5) (width 0.2) (layer "F.Cu") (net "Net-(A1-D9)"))
 (segment (start 147.424925 116.144365) (end 147.424925 117.055635) (width 0.2) (layer "F.Cu") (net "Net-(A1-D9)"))
 (segment (start 94.364925 118.1) (end 90.354925 114.09) (width 0.2) (layer "F.Cu") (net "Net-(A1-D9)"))
 (segment (start 144.884925 115.5) (end 146.78056 115.5) (width 0.2) (layer "F.Cu") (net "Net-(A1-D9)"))
 (segment (start 147.424925 117.055635) (end 146.38056 118.1) (width 0.2) (layer "F.Cu") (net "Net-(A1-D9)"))
 (segment (start 146.38056 118.1) (end 94.364925 118.1) (width 0.2) (layer "F.Cu") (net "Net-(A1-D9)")))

